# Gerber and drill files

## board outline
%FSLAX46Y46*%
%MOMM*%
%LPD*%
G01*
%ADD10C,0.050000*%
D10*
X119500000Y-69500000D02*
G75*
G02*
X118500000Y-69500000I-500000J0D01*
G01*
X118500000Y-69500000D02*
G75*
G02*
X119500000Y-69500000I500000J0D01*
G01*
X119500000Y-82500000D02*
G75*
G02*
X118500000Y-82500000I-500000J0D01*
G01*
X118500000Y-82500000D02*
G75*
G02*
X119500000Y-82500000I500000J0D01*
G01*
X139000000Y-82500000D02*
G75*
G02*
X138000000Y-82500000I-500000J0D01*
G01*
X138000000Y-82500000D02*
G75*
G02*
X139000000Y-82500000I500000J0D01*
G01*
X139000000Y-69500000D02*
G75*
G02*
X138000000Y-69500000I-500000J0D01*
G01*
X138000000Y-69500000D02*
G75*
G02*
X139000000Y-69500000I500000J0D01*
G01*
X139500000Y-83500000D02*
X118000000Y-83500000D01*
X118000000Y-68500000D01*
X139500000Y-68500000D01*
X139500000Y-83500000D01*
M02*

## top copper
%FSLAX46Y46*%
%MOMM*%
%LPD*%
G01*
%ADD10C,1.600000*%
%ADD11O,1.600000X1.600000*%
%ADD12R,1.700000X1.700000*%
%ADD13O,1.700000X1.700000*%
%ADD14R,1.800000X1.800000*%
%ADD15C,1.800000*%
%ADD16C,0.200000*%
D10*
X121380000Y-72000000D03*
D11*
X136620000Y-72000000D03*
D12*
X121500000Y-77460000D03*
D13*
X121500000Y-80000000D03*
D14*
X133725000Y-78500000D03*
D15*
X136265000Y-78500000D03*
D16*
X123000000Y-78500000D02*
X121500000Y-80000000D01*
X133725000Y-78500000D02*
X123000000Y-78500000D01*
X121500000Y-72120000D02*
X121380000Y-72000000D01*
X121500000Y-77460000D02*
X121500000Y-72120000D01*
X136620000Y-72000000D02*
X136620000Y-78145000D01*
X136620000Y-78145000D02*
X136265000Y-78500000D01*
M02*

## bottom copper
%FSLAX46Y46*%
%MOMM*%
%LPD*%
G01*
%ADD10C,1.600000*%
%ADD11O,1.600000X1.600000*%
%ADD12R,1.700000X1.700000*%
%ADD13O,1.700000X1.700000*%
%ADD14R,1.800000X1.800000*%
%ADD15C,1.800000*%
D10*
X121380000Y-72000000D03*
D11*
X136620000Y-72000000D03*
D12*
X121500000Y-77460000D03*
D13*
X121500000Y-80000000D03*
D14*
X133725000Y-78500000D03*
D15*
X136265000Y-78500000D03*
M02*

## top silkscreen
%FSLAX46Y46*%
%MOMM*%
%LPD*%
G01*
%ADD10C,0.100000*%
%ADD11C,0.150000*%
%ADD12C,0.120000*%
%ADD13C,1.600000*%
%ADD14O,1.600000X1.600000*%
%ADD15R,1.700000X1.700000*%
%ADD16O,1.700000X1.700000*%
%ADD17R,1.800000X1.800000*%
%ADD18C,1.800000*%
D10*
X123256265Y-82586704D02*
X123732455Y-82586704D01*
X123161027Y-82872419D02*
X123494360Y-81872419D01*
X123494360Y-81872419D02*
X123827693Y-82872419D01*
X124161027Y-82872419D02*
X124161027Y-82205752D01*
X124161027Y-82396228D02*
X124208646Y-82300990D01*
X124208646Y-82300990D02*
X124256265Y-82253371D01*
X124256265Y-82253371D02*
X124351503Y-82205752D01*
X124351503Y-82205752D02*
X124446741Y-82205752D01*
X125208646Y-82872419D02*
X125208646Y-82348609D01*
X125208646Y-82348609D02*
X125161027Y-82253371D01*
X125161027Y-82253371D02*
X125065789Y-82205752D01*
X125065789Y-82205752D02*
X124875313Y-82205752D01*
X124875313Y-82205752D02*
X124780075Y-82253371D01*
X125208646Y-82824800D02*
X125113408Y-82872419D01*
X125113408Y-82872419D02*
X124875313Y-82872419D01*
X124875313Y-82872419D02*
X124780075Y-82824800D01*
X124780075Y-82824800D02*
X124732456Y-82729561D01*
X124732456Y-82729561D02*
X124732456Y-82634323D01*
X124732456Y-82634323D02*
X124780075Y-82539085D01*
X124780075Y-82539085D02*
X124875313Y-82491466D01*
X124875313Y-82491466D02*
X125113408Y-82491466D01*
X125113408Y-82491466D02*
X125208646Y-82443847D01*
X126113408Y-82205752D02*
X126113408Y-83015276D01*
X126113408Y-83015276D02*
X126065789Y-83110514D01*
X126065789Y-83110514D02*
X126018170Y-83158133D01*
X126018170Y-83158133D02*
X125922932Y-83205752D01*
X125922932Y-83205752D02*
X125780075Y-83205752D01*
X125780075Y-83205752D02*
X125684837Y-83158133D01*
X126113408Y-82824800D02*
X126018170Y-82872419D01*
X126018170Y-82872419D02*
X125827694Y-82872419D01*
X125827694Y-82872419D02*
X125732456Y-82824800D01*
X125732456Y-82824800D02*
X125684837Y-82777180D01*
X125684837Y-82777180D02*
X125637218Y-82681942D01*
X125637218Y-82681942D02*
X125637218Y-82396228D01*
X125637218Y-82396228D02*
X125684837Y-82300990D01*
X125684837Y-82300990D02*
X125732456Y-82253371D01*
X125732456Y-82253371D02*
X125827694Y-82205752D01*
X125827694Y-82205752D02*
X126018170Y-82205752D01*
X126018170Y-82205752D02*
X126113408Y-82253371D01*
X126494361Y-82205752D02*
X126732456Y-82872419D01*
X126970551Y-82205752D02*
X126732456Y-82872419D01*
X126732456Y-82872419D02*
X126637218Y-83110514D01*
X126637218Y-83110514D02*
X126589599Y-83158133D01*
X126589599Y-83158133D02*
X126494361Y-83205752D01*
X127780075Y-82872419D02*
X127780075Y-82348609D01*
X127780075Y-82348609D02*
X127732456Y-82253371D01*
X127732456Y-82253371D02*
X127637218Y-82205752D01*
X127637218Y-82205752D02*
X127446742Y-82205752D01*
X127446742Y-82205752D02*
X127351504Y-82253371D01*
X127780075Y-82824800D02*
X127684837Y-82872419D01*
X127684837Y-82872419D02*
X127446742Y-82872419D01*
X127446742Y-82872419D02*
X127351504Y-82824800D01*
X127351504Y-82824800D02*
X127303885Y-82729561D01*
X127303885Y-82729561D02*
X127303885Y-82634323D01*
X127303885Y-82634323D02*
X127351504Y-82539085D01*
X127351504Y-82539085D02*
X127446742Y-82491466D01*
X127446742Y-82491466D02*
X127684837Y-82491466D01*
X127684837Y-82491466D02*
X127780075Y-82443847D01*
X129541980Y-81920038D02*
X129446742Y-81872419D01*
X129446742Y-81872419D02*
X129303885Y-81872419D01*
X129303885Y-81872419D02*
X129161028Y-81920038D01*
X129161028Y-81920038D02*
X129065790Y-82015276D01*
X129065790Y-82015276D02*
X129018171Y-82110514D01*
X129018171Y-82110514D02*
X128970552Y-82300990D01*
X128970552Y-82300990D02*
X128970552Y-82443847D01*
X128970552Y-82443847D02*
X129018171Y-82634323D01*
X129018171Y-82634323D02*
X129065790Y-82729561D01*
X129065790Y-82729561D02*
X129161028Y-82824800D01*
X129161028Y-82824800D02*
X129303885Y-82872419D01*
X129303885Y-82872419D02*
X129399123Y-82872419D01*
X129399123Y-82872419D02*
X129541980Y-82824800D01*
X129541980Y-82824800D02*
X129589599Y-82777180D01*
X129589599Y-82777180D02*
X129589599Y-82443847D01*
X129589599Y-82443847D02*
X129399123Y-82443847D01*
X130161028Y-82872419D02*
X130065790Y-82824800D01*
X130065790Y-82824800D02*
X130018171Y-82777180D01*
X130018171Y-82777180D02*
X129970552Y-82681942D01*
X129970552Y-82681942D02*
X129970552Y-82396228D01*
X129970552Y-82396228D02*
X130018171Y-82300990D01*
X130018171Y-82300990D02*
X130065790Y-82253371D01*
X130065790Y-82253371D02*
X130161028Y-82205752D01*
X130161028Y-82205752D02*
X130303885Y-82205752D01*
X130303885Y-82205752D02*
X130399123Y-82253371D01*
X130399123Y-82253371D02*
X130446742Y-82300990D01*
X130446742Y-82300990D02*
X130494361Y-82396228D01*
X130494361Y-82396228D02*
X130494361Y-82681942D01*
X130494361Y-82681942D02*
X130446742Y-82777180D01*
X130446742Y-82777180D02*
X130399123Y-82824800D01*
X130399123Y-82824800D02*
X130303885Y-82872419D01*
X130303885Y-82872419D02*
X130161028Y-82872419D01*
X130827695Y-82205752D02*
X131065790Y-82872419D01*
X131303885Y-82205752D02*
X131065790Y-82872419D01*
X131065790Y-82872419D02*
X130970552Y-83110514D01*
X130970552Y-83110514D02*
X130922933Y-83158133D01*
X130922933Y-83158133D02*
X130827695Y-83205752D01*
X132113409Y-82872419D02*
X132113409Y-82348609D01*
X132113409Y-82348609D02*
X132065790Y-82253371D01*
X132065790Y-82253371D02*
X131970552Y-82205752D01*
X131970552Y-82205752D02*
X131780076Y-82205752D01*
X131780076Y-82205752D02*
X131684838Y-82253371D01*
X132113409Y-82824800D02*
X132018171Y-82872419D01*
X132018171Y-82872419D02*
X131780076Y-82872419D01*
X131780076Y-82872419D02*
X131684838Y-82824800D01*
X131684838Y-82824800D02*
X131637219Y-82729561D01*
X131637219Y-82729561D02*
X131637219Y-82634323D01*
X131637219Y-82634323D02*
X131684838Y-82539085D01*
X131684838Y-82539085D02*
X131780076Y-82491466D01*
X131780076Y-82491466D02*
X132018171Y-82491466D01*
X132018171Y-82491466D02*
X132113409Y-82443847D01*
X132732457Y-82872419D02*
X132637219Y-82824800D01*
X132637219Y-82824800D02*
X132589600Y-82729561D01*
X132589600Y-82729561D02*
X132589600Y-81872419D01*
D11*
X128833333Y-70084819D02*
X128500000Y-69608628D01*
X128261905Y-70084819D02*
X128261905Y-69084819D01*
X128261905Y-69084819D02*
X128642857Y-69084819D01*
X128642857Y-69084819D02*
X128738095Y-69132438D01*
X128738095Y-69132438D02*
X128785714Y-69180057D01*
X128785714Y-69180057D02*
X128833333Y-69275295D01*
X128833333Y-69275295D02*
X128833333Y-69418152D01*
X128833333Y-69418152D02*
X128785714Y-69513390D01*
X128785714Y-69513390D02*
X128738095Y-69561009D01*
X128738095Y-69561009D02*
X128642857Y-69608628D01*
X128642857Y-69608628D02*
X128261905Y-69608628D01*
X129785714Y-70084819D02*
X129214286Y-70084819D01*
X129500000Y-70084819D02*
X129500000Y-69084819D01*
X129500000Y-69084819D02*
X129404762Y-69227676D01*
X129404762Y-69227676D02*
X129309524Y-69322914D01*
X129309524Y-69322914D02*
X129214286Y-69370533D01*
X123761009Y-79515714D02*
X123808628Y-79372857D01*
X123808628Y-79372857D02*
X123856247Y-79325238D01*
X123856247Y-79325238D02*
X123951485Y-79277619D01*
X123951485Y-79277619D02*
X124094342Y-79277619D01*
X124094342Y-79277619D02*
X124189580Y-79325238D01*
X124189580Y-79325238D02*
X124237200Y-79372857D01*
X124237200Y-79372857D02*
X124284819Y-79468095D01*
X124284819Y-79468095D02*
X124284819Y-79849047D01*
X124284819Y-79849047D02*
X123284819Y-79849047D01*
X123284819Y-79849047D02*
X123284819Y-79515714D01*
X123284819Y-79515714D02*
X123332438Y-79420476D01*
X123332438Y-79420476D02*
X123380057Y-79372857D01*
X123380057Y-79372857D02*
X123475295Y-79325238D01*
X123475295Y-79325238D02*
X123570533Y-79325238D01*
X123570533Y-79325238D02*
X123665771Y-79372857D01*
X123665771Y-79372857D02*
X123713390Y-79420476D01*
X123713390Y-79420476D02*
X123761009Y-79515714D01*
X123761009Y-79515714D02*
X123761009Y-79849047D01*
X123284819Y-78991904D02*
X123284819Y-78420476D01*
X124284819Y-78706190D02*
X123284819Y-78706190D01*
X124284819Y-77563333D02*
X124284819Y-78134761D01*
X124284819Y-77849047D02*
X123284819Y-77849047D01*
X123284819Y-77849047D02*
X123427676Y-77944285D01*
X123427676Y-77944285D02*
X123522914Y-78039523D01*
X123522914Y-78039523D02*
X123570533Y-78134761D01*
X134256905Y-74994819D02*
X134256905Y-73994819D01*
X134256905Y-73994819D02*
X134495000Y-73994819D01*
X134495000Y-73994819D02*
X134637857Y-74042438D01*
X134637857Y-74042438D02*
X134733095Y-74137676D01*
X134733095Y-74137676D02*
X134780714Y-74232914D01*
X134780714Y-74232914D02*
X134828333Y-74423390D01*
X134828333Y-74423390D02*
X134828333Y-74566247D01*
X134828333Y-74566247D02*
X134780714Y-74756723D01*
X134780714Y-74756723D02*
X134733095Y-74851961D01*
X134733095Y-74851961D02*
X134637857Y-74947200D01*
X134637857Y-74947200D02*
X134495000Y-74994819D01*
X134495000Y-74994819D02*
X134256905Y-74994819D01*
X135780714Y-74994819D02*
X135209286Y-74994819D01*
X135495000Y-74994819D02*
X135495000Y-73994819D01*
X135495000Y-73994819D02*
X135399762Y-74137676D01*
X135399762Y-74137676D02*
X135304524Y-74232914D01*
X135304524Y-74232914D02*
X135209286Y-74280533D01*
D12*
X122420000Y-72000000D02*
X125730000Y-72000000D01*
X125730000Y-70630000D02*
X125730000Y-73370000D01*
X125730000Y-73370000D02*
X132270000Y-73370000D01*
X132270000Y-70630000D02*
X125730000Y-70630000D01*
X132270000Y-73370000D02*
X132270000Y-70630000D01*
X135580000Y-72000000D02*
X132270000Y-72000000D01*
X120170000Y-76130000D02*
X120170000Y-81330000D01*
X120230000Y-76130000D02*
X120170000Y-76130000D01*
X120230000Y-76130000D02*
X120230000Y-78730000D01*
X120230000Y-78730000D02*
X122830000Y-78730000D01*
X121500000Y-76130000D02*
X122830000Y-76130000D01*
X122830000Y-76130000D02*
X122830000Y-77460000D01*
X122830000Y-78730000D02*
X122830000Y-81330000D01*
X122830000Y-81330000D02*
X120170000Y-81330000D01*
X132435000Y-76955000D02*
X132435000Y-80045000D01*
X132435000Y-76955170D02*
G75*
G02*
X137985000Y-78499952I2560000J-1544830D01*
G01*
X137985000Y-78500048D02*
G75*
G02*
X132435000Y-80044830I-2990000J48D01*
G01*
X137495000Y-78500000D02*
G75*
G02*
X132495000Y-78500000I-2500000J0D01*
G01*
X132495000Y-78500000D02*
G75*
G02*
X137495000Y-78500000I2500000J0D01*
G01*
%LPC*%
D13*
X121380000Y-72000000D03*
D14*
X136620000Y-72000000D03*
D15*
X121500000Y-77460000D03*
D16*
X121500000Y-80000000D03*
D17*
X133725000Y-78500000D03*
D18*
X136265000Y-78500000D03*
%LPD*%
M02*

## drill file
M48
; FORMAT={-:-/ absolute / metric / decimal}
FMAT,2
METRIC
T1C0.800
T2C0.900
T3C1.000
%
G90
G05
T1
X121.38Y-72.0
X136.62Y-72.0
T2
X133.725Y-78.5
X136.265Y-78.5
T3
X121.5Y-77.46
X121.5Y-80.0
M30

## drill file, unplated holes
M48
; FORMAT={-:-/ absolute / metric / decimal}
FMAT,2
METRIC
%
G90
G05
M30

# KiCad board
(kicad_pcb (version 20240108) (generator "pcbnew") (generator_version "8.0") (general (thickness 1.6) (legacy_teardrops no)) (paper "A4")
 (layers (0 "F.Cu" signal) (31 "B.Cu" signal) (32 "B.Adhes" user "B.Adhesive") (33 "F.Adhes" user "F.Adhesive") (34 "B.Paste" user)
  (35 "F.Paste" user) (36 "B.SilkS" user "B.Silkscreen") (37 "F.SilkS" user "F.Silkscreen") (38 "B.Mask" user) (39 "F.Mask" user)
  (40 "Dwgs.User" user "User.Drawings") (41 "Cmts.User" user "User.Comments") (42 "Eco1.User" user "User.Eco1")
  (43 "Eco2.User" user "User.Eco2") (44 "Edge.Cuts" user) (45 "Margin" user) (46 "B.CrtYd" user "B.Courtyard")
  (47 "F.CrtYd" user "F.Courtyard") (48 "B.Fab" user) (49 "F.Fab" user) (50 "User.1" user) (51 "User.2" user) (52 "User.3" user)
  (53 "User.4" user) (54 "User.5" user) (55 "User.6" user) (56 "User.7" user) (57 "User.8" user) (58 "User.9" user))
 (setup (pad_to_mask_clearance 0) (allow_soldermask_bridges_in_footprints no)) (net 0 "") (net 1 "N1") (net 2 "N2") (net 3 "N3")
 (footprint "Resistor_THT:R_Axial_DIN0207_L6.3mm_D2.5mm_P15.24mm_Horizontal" (layer "F.Cu") (at 121.38 72)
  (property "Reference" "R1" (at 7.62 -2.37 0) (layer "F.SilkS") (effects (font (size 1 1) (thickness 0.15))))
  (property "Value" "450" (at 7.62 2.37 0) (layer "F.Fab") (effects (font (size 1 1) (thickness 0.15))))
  (fp_line (start 1.04 0) (end 4.35 0) (stroke (width 0.12) (type solid)) (layer "F.SilkS"))
  (fp_line (start 4.35 -1.37) (end 4.35 1.37) (stroke (width 0.12) (type solid)) (layer "F.SilkS"))
  (fp_line (start 4.35 1.37) (end 10.89 1.37) (stroke (width 0.12) (type solid)) (layer "F.SilkS"))
  (fp_line (start 10.89 -1.37) (end 4.35 -1.37) (stroke (width 0.12) (type solid)) (layer "F.SilkS"))
  (fp_line (start 10.89 1.37) (end 10.89 -1.37) (stroke (width 0.12) (type solid)) (layer "F.SilkS"))
  (fp_line (start 14.2 0) (end 10.89 0) (stroke (width 0.12) (type solid)) (layer "F.SilkS"))
  (pad "1" thru_hole circle (at 0 0) (size 1.6 1.6) (drill 0.8) (layers "*.Cu" "*.Mask") (remove_unused_layers no) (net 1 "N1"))
  (pad "2" thru_hole oval (at 15.24 0) (size 1.6 1.6) (drill 0.8) (layers "*.Cu" "*.Mask") (remove_unused_layers no) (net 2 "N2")))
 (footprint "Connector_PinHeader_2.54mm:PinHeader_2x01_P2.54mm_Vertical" (layer "F.Cu") (at 121.5 77.46 -90)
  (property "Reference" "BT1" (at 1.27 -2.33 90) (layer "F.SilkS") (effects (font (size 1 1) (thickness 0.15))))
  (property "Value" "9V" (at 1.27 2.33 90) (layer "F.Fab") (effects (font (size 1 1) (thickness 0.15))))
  (fp_line (start -1.33 1.33) (end 3.87 1.33) (stroke (width 0.12) (type solid)) (layer "F.SilkS"))
  (fp_line (start -1.33 1.27) (end -1.33 1.33) (stroke (width 0.12) (type solid)) (layer "F.SilkS"))
  (fp_line (start -1.33 1.27) (end 1.27 1.27) (stroke (width 0.12) (type solid)) (layer "F.SilkS"))
  (fp_line (start 1.27 1.27) (end 1.27 -1.33) (stroke (width 0.12) (type solid)) (layer "F.SilkS"))
  (fp_line (start -1.33 0) (end -1.33 -1.33) (stroke (width 0.12) (type solid)) (layer "F.SilkS"))
  (fp_line (start -1.33 -1.33) (end 0 -1.33) (stroke (width 0.12) (type solid)) (layer "F.SilkS"))
  (fp_line (start 1.27 -1.33) (end 3.87 -1.33) (stroke (width 0.12) (type solid)) (layer "F.SilkS"))
  (fp_line (start 3.87 -1.33) (end 3.87 1.33) (stroke (width 0.12) (type solid)) (layer "F.SilkS"))
  (pad "1" thru_hole rect (at 0 0 270) (size 1.7 1.7) (drill 1) (layers "*.Cu" "*.Mask") (remove_unused_layers no) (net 1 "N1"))
  (pad "2" thru_hole oval (at 2.54 0 270) (size 1.7 1.7) (drill 1) (layers "*.Cu" "*.Mask") (remove_unused_layers no) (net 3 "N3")))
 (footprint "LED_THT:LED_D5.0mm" (layer "F.Cu") (at 133.725 78.5)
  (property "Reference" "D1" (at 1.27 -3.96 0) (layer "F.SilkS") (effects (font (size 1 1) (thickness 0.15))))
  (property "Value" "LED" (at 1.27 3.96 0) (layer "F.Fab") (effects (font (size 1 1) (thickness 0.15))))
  (fp_line (start -1.29 -1.545) (end -1.29 1.545) (stroke (width 0.12) (type solid)) (layer "F.SilkS"))
  (fp_arc (start -1.29 -1.54483) (mid 2.071756 -2.880501) (end 4.26 -0.000048) (stroke (width 0.12) (type solid)) (layer "F.SilkS"))
  (fp_arc (start 4.26 0.000048) (mid 2.071756 2.880501) (end -1.29 1.54483) (stroke (width 0.12) (type solid)) (layer "F.SilkS"))
  (fp_circle (center 1.27 0) (end 3.77 0) (stroke (width 0.12) (type solid)) (fill none) (layer "F.SilkS"))
  (pad "1" thru_hole rect (at 0 0) (size 1.8 1.8) (drill 0.9) (layers "*.Cu" "*.Mask") (remove_unused_layers no) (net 3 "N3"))
  (pad "2" thru_hole circle (at 2.54 0) (size 1.8 1.8) (drill 0.9) (layers "*.Cu" "*.Mask") (remove_unused_layers no) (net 2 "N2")))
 (gr_circle (center 119 82.5) (end 118.5 82.5) (stroke (width 0.05) (type default)) (fill none) (layer "Edge.Cuts"))
 (gr_circle (center 138.5 69.5) (end 139 69.5) (stroke (width 0.05) (type default)) (fill none) (layer "Edge.Cuts"))
 (gr_circle (center 119 69.5) (end 118.5 69.5) (stroke (width 0.05) (type default)) (fill none) (layer "Edge.Cuts"))
 (gr_poly
  (pts (xy 139.5 68.5) (xy 139.5 83.5) (xy 118 83.5) (xy 118 68.5)) (stroke (width 0.05) (type solid)) (fill none) (layer "Edge.Cuts"))
 (gr_circle (center 138.5 82.5) (end 139 82.5) (stroke (width 0.05) (type default)) (fill none) (layer "Edge.Cuts"))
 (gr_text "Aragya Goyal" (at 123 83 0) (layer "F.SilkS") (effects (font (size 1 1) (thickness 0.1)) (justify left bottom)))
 (segment (start 123 78.5) (end 121.5 80) (width 0.2) (layer "F.Cu") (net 3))
 (segment (start 133.725 78.5) (end 123 78.5) (width 0.2) (layer "F.Cu") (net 3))
 (segment (start 121.5 72.12) (end 121.38 72) (width 0.2) (layer "F.Cu") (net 1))
 (segment (start 121.5 77.46) (end 121.5 72.12) (width 0.2) (layer "F.Cu") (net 1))
 (segment (start 136.62 72) (end 136.62 78.145) (width 0.2) (layer "F.Cu") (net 2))
 (segment (start 136.62 78.145) (end 136.265 78.5) (width 0.2) (layer "F.Cu") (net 2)))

